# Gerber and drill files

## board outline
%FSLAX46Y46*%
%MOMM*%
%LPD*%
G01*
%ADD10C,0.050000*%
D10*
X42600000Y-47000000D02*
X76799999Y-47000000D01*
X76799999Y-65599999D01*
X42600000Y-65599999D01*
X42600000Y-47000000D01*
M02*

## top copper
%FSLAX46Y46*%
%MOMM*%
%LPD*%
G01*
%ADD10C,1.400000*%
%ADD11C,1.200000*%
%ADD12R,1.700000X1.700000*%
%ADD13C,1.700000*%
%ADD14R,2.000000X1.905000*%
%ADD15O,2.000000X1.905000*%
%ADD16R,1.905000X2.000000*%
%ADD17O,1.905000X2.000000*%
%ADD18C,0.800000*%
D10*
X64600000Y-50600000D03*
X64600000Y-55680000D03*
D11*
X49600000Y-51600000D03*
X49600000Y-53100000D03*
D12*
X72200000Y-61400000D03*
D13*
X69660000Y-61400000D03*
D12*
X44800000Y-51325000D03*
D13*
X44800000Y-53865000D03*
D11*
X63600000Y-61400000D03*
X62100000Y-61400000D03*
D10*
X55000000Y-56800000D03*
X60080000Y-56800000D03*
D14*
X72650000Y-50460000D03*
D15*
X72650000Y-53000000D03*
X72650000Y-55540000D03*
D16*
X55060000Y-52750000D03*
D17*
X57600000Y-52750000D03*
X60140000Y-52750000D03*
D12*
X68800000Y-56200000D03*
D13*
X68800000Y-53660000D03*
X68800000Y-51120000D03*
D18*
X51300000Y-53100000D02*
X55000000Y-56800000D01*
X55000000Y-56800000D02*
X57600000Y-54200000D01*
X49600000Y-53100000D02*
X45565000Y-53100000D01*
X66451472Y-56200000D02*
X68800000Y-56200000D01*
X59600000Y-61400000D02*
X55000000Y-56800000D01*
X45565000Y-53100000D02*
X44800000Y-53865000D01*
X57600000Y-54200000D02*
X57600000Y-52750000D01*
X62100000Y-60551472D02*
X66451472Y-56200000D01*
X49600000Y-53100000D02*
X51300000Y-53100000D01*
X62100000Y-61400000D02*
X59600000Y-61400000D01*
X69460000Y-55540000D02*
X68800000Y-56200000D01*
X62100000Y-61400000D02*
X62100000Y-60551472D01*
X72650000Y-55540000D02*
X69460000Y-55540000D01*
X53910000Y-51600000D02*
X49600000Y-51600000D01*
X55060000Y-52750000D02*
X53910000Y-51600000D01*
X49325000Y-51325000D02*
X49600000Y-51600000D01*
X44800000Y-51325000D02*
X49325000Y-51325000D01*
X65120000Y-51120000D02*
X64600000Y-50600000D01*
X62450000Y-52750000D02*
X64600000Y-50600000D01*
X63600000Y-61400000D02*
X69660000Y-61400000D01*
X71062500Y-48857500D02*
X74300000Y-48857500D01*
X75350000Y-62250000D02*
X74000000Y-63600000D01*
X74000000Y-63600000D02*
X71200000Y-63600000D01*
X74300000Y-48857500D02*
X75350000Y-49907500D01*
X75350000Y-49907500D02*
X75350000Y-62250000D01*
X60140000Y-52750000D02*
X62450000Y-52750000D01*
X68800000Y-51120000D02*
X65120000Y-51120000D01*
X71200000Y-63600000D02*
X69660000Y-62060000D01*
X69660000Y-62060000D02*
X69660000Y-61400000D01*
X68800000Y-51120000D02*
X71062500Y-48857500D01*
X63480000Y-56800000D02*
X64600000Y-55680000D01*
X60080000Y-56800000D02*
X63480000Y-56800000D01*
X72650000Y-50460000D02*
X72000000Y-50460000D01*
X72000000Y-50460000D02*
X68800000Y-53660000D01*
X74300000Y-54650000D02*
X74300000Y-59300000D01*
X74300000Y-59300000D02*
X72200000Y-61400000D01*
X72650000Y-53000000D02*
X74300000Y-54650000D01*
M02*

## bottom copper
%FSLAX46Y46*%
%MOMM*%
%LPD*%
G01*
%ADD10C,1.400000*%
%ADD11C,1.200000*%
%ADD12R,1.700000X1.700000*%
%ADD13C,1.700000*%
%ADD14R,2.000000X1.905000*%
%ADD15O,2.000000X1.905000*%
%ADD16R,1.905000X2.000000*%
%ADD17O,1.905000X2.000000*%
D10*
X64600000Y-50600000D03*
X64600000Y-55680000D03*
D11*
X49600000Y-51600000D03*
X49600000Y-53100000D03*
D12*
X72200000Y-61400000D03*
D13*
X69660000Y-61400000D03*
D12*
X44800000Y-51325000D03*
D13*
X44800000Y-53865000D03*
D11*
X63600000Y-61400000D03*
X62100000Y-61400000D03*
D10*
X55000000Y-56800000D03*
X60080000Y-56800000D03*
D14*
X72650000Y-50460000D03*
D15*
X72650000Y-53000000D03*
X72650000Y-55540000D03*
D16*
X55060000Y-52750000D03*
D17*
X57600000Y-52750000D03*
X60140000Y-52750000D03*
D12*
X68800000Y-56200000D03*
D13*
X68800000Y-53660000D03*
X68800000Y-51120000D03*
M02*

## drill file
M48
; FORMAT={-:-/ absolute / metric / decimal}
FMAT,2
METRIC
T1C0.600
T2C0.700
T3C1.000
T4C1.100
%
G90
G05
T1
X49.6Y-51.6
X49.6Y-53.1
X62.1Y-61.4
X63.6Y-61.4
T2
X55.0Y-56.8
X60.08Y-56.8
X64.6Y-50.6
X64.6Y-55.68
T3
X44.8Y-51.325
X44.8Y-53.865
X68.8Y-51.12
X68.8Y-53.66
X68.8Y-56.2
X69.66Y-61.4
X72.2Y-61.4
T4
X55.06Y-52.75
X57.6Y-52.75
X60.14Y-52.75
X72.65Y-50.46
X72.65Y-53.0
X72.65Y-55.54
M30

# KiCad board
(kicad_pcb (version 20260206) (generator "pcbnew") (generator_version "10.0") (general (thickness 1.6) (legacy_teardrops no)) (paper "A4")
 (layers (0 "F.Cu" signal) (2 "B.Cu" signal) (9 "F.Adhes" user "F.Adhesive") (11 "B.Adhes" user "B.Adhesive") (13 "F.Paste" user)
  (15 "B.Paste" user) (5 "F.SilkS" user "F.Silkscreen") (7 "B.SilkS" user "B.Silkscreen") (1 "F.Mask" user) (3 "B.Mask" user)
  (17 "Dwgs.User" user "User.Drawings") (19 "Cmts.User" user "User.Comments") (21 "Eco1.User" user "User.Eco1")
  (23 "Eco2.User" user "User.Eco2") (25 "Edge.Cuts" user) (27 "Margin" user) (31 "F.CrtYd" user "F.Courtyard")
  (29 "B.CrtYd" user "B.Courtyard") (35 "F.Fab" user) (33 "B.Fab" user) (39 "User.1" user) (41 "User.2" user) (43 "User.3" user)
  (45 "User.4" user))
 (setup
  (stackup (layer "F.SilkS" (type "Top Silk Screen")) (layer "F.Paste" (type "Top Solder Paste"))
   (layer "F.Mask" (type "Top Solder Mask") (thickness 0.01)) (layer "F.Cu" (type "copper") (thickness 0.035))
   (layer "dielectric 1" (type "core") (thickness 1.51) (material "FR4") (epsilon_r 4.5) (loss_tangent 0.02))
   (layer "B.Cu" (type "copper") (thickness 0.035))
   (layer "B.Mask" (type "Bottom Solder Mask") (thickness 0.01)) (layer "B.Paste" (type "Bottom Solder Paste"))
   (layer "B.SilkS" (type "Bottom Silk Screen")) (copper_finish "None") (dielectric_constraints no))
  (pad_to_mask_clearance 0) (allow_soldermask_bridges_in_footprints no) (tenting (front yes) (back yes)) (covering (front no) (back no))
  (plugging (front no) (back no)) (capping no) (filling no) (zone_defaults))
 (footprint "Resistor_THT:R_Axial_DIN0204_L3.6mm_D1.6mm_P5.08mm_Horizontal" (layer "F.Cu") (at 64.6 50.6 -90)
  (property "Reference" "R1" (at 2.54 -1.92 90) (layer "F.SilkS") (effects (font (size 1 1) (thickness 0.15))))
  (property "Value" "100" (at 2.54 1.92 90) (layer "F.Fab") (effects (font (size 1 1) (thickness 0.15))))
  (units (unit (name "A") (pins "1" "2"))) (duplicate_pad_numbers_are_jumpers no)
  (pad "1" thru_hole circle (at 0 0 270) (size 1.4 1.4) (drill 0.7) (layers "*.Cu" "*.Mask") (remove_unused_layers no) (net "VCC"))
  (pad "2" thru_hole circle (at 5.08 0 270) (size 1.4 1.4) (drill 0.7) (layers "*.Cu" "*.Mask") (remove_unused_layers no) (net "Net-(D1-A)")))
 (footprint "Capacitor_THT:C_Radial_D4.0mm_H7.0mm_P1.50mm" (layer "F.Cu") (at 49.6 51.6 -90)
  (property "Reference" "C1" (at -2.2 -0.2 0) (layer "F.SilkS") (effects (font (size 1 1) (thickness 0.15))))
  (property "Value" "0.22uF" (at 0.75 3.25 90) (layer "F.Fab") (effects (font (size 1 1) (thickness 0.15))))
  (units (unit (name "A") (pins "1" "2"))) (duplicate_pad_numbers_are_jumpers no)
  (pad "1" thru_hole circle (at 0 0 270) (size 1.2 1.2) (drill 0.6) (layers "*.Cu" "*.Mask") (remove_unused_layers no) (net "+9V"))
  (pad "2" thru_hole circle (at 1.5 0 270) (size 1.2 1.2) (drill 0.6) (layers "*.Cu" "*.Mask") (remove_unused_layers no) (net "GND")))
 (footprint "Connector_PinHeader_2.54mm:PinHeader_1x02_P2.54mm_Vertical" (layer "F.Cu") (at 72.2 61.4 -90)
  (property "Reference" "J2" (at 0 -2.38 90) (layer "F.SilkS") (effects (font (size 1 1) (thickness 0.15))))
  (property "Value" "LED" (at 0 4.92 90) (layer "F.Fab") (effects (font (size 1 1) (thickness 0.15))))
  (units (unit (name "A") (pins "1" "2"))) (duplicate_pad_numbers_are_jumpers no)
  (pad "1" thru_hole rect (at 0 0 270) (size 1.7 1.7) (drill 1) (layers "*.Cu" "*.Mask") (remove_unused_layers no) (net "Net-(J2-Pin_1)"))
  (pad "2" thru_hole circle (at 0 2.54 270) (size 1.7 1.7) (drill 1) (layers "*.Cu" "*.Mask") (remove_unused_layers no) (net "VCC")))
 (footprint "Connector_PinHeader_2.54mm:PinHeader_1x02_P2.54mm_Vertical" (layer "F.Cu") (at 44.8 51.325)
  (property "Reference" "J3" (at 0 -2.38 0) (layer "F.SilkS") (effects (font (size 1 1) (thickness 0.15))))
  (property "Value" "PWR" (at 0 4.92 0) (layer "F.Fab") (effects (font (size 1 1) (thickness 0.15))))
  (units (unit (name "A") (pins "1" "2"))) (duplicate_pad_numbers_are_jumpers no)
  (pad "1" thru_hole rect (at 0 0) (size 1.7 1.7) (drill 1) (layers "*.Cu" "*.Mask") (remove_unused_layers no) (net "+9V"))
  (pad "2" thru_hole circle (at 0 2.54) (size 1.7 1.7) (drill 1) (layers "*.Cu" "*.Mask") (remove_unused_layers no) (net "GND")))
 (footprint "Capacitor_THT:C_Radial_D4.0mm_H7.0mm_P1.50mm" (layer "F.Cu") (at 63.6 61.4 180)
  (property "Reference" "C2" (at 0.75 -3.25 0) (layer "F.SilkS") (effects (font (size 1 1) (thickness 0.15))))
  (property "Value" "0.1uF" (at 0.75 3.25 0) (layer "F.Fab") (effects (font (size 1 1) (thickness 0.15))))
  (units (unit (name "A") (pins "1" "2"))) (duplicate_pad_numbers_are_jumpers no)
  (pad "1" thru_hole circle (at 0 0 180) (size 1.2 1.2) (drill 0.6) (layers "*.Cu" "*.Mask") (remove_unused_layers no) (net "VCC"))
  (pad "2" thru_hole circle (at 1.5 0 180) (size 1.2 1.2) (drill 0.6) (layers "*.Cu" "*.Mask") (remove_unused_layers no) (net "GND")))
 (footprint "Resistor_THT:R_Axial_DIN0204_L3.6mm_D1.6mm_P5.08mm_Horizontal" (layer "F.Cu") (at 55 56.8)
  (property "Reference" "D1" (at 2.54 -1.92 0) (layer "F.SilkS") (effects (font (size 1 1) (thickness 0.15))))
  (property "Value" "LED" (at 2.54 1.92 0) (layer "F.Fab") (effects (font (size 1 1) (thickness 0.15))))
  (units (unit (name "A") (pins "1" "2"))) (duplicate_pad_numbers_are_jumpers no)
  (pad "1" thru_hole circle (at 0 0) (size 1.4 1.4) (drill 0.7) (layers "*.Cu" "*.Mask") (remove_unused_layers no) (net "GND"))
  (pad "2" thru_hole circle (at 5.08 0) (size 1.4 1.4) (drill 0.7) (layers "*.Cu" "*.Mask") (remove_unused_layers no) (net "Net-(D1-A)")))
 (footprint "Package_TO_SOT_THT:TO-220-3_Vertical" (layer "F.Cu") (at 72.65 50.46 -90)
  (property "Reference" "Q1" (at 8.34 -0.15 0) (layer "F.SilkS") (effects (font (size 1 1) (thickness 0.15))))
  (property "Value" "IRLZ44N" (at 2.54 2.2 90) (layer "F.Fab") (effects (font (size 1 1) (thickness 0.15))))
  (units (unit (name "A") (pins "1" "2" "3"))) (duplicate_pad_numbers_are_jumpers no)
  (pad "1" thru_hole rect (at 0 0 270) (size 1.905 2) (drill 1.1) (layers "*.Cu" "*.Mask") (remove_unused_layers no) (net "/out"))
  (pad "2" thru_hole oval (at 2.54 0 270) (size 1.905 2) (drill 1.1) (layers "*.Cu" "*.Mask") (remove_unused_layers no)
   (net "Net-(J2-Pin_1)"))
  (pad "3" thru_hole oval (at 5.08 0 270) (size 1.905 2) (drill 1.1) (layers "*.Cu" "*.Mask") (remove_unused_layers no) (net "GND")))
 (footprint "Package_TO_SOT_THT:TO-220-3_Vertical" (layer "F.Cu") (at 55.06 52.75)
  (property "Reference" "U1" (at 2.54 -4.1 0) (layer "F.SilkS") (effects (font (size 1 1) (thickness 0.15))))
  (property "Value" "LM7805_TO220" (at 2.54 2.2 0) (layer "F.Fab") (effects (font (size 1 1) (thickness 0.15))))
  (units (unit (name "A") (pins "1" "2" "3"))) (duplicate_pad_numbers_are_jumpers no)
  (pad "1" thru_hole rect (at 0 0) (size 1.905 2) (drill 1.1) (layers "*.Cu" "*.Mask") (remove_unused_layers no) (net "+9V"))
  (pad "2" thru_hole oval (at 2.54 0) (size 1.905 2) (drill 1.1) (layers "*.Cu" "*.Mask") (remove_unused_layers no) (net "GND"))
  (pad "3" thru_hole oval (at 5.08 0) (size 1.905 2) (drill 1.1) (layers "*.Cu" "*.Mask") (remove_unused_layers no) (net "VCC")))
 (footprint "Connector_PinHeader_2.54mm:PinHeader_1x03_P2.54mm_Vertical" (layer "F.Cu") (at 68.8 56.2 180)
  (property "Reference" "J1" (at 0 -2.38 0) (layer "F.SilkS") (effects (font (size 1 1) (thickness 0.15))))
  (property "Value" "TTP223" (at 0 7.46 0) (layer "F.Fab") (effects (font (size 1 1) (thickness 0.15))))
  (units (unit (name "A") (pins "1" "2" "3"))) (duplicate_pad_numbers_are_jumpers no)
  (pad "1" thru_hole rect (at 0 0 180) (size 1.7 1.7) (drill 1) (layers "*.Cu" "*.Mask") (remove_unused_layers no) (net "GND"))
  (pad "2" thru_hole circle (at 0 2.54 180) (size 1.7 1.7) (drill 1) (layers "*.Cu" "*.Mask") (remove_unused_layers no) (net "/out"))
  (pad "3" thru_hole circle (at 0 5.08 180) (size 1.7 1.7) (drill 1) (layers "*.Cu" "*.Mask") (remove_unused_layers no) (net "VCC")))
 (gr_rect (start 42.6 47) (end 76.799999 65.599999) (stroke (width 0.05) (type solid)) (fill no) (layer "Edge.Cuts"))
 (segment (start 51.3 53.1) (end 55 56.8) (width 0.8) (layer "F.Cu") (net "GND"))
 (segment (start 55 56.8) (end 57.6 54.2) (width 0.8) (layer "F.Cu") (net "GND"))
 (segment (start 49.6 53.1) (end 45.565 53.1) (width 0.8) (layer "F.Cu") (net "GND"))
 (segment (start 66.451472 56.2) (end 68.8 56.2) (width 0.8) (layer "F.Cu") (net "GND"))
 (segment (start 59.6 61.4) (end 55 56.8) (width 0.8) (layer "F.Cu") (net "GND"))
 (segment (start 45.565 53.1) (end 44.8 53.865) (width 0.8) (layer "F.Cu") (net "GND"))
 (segment (start 57.6 54.2) (end 57.6 52.75) (width 0.8) (layer "F.Cu") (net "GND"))
 (segment (start 62.1 60.551472) (end 66.451472 56.2) (width 0.8) (layer "F.Cu") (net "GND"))
 (segment (start 49.6 53.1) (end 51.3 53.1) (width 0.8) (layer "F.Cu") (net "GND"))
 (segment (start 62.1 61.4) (end 59.6 61.4) (width 0.8) (layer "F.Cu") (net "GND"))
 (segment (start 69.46 55.54) (end 68.8 56.2) (width 0.8) (layer "F.Cu") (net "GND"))
 (segment (start 62.1 61.4) (end 62.1 60.551472) (width 0.8) (layer "F.Cu") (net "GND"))
 (segment (start 72.65 55.54) (end 69.46 55.54) (width 0.8) (layer "F.Cu") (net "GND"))
 (segment (start 53.91 51.6) (end 49.6 51.6) (width 0.8) (layer "F.Cu") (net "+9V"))
 (segment (start 55.06 52.75) (end 53.91 51.6) (width 0.8) (layer "F.Cu") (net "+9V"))
 (segment (start 49.325 51.325) (end 49.6 51.6) (width 0.8) (layer "F.Cu") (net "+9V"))
 (segment (start 44.8 51.325) (end 49.325 51.325) (width 0.8) (layer "F.Cu") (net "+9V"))
 (segment (start 65.12 51.12) (end 64.6 50.6) (width 0.8) (layer "F.Cu") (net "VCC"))
 (segment (start 62.45 52.75) (end 64.6 50.6) (width 0.8) (layer "F.Cu") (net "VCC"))
 (segment (start 63.6 61.4) (end 69.66 61.4) (width 0.8) (layer "F.Cu") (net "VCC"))
 (segment (start 71.0625 48.8575) (end 74.3 48.8575) (width 0.8) (layer "F.Cu") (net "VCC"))
 (segment (start 75.35 62.25) (end 74 63.6) (width 0.8) (layer "F.Cu") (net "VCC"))
 (segment (start 74 63.6) (end 71.2 63.6) (width 0.8) (layer "F.Cu") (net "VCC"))
 (segment (start 74.3 48.8575) (end 75.35 49.9075) (width 0.8) (layer "F.Cu") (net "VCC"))
 (segment (start 75.35 49.9075) (end 75.35 62.25) (width 0.8) (layer "F.Cu") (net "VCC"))
 (segment (start 60.14 52.75) (end 62.45 52.75) (width 0.8) (layer "F.Cu") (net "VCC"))
 (segment (start 68.8 51.12) (end 65.12 51.12) (width 0.8) (layer "F.Cu") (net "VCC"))
 (segment (start 71.2 63.6) (end 69.66 62.06) (width 0.8) (layer "F.Cu") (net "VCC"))
 (segment (start 69.66 62.06) (end 69.66 61.4) (width 0.8) (layer "F.Cu") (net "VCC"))
 (segment (start 68.8 51.12) (end 71.0625 48.8575) (width 0.8) (layer "F.Cu") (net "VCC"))
 (segment (start 63.48 56.8) (end 64.6 55.68) (width 0.8) (layer "F.Cu") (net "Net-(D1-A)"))
 (segment (start 60.08 56.8) (end 63.48 56.8) (width 0.8) (layer "F.Cu") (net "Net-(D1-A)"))
 (segment (start 72.65 50.46) (end 72 50.46) (width 0.8) (layer "F.Cu") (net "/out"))
 (segment (start 72 50.46) (end 68.8 53.66) (width 0.8) (layer "F.Cu") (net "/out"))
 (segment (start 74.3 54.65) (end 74.3 59.3) (width 0.8) (layer "F.Cu") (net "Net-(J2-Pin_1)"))
 (segment (start 74.3 59.3) (end 72.2 61.4) (width 0.8) (layer "F.Cu") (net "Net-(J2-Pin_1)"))
 (segment (start 72.65 53) (end 74.3 54.65) (width 0.8) (layer "F.Cu") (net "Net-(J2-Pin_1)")))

